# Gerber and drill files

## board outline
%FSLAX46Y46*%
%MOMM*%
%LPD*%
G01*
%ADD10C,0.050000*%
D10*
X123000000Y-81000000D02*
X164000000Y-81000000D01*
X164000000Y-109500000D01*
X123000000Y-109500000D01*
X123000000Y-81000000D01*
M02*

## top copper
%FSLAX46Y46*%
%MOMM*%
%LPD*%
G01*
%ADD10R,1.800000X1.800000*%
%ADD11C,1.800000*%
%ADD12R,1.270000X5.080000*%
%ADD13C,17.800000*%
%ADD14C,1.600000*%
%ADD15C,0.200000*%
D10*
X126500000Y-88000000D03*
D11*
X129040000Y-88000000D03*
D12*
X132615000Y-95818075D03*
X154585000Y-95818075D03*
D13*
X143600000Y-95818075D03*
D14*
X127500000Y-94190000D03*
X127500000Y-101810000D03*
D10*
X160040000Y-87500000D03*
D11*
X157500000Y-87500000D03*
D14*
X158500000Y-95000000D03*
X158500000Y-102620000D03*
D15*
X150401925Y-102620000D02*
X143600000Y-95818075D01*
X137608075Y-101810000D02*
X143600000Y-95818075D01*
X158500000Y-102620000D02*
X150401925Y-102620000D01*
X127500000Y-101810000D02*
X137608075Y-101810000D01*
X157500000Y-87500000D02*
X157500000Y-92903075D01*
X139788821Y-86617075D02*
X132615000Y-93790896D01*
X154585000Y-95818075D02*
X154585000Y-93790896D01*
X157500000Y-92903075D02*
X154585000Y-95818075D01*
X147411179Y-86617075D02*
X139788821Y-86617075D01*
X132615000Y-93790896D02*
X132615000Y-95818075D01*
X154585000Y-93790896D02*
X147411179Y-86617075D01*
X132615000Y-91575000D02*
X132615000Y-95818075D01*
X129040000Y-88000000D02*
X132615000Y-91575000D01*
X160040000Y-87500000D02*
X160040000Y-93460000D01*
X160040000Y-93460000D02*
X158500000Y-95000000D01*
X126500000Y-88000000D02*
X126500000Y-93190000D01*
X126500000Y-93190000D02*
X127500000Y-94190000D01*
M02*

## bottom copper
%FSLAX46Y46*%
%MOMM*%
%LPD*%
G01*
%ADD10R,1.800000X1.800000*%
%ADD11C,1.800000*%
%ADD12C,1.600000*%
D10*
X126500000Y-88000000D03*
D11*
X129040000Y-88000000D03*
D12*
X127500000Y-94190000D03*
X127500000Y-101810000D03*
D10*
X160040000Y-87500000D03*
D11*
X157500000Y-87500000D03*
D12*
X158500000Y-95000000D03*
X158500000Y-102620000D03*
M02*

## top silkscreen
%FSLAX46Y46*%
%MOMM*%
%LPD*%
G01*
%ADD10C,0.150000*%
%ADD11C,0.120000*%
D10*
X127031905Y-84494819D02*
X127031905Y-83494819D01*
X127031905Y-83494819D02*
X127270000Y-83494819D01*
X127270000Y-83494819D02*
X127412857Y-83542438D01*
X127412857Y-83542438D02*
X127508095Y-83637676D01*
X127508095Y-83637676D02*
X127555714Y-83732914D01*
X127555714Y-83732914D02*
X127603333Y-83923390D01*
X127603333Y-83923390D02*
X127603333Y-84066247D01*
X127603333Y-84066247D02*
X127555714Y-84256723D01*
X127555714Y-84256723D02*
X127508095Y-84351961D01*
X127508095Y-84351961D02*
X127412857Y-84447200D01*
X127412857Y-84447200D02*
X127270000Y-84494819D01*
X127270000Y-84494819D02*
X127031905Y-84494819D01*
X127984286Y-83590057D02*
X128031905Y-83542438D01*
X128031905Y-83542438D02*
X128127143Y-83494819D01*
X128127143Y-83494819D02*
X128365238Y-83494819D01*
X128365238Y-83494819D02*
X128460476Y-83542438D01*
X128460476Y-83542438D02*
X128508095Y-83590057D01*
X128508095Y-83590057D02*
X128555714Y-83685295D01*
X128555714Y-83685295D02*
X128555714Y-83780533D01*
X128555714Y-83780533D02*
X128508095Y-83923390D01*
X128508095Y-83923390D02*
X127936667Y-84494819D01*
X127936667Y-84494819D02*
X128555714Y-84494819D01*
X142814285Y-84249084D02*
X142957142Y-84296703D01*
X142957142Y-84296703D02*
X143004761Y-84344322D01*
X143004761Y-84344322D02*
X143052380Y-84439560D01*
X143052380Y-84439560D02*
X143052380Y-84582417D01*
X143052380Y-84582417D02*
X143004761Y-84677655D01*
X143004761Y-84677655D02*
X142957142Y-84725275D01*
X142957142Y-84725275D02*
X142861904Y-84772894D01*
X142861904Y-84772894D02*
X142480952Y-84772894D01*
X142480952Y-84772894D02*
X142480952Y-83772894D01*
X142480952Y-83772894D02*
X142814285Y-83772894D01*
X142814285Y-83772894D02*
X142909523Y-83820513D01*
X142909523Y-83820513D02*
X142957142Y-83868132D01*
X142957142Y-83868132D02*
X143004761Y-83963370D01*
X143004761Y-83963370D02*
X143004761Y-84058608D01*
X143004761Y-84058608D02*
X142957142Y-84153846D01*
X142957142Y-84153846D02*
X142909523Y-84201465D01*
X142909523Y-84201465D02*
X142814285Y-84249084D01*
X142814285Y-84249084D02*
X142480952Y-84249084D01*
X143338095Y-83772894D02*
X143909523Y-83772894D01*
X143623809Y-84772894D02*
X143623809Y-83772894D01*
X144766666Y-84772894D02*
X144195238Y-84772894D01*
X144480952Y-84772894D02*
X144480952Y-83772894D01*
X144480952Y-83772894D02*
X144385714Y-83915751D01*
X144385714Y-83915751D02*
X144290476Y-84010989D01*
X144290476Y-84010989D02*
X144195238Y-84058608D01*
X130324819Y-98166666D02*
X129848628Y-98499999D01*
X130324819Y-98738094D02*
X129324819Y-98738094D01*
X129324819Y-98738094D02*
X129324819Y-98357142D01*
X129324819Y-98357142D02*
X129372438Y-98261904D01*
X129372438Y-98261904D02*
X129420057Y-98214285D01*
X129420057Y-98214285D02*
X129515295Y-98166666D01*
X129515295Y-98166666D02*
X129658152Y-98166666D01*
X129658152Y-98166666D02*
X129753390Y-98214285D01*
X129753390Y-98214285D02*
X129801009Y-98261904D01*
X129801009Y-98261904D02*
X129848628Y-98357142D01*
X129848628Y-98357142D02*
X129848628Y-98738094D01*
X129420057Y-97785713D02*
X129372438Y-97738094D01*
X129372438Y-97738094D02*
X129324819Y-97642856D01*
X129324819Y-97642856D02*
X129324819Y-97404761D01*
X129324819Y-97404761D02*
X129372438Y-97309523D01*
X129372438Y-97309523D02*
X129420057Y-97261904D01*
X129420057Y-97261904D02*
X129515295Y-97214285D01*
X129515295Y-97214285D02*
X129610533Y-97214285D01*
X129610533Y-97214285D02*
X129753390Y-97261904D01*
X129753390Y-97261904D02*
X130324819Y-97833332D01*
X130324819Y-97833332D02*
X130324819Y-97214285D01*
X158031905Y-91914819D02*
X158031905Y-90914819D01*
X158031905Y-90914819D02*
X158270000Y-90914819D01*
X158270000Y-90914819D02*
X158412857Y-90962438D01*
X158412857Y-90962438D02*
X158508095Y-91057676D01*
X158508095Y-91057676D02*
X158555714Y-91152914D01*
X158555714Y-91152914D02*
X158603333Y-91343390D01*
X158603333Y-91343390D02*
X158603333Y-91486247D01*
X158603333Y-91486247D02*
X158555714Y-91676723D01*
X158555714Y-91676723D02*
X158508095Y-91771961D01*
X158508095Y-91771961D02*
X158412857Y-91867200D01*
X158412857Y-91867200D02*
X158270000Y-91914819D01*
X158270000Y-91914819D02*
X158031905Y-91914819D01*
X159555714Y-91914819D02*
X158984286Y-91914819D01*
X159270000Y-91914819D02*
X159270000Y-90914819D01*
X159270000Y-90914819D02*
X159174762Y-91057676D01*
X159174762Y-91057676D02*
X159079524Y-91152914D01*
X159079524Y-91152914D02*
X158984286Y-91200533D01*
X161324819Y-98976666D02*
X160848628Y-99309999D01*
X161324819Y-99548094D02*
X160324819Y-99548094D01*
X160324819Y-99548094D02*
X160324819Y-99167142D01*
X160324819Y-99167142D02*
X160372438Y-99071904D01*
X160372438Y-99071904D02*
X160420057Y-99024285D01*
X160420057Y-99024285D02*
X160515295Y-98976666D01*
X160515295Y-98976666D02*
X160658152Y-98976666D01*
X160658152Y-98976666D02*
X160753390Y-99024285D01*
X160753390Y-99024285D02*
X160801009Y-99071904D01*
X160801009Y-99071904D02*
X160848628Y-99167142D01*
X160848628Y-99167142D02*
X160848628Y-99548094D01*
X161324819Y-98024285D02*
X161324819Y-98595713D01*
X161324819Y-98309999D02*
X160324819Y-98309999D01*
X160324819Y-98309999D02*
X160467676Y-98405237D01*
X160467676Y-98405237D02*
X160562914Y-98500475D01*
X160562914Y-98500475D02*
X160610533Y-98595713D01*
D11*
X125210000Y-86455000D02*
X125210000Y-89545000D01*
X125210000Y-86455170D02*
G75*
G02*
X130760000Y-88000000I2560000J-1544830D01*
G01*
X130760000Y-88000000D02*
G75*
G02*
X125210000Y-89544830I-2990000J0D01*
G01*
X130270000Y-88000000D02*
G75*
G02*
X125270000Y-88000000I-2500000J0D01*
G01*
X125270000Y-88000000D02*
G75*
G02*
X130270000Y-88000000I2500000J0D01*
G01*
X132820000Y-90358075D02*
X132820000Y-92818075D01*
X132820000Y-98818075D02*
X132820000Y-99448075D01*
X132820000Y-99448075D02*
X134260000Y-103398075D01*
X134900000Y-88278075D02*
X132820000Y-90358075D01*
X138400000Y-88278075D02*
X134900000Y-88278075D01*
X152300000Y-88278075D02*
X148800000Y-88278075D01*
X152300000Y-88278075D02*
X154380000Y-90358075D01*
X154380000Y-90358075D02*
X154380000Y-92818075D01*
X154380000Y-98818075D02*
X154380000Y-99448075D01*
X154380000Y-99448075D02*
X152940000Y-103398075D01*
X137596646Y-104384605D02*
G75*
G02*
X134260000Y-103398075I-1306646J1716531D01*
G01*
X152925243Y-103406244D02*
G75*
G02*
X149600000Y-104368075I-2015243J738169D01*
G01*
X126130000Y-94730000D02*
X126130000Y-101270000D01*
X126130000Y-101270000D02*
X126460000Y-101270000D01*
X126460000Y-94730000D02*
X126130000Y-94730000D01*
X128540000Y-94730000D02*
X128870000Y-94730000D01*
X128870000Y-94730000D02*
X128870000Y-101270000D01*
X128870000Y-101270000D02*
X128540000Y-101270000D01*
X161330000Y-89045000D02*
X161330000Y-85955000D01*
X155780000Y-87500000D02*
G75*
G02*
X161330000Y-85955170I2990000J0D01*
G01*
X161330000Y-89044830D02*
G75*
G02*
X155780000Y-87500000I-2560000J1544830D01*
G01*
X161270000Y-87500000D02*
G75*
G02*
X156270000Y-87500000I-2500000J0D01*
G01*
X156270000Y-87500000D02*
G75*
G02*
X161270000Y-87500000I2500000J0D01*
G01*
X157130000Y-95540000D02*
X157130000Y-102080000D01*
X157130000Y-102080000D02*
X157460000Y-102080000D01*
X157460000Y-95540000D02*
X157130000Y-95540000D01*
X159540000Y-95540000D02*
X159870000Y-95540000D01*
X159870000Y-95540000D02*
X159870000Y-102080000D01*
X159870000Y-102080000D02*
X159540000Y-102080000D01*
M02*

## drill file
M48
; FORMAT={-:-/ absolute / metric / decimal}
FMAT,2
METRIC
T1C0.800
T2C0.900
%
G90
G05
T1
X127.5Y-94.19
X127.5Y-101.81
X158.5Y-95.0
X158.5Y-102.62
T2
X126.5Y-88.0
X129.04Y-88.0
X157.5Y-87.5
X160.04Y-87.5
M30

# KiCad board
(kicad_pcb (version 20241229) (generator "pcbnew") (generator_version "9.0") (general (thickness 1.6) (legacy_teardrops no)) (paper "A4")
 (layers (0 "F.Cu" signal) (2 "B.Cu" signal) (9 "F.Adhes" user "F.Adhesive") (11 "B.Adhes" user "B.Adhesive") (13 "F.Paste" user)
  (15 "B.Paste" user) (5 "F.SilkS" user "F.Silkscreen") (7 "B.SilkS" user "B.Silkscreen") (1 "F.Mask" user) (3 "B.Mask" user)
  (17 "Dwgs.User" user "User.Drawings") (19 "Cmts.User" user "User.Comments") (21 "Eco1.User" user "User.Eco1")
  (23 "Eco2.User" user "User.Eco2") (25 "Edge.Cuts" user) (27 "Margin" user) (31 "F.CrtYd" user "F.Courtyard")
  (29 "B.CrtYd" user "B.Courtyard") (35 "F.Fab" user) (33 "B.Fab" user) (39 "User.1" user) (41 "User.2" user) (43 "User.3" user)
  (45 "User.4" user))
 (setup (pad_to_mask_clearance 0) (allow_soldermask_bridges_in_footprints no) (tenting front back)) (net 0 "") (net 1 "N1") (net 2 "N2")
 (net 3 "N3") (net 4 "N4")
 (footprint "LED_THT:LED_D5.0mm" (layer "F.Cu") (at 126.5 88)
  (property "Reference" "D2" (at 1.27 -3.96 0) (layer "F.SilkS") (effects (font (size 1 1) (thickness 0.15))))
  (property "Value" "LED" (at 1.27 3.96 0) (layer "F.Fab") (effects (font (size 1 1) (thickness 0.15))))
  (fp_line (start -1.29 -1.545) (end -1.29 1.545) (stroke (width 0.12) (type solid)) (layer "F.SilkS"))
  (fp_arc (start -1.29 -1.54483) (mid 2.071779 -2.880495) (end 4.26 0) (stroke (width 0.12) (type solid)) (layer "F.SilkS"))
  (fp_arc (start 4.26 0) (mid 2.071779 2.880495) (end -1.29 1.54483) (stroke (width 0.12) (type solid)) (layer "F.SilkS"))
  (fp_circle (center 1.27 0) (end 3.77 0) (stroke (width 0.12) (type solid)) (fill no) (layer "F.SilkS"))
  (pad "1" thru_hole rect (at 0 0) (size 1.8 1.8) (drill 0.9) (layers "*.Cu" "*.Mask") (remove_unused_layers no) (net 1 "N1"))
  (pad "2" thru_hole circle (at 2.54 0) (size 1.8 1.8) (drill 0.9) (layers "*.Cu" "*.Mask") (remove_unused_layers no) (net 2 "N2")))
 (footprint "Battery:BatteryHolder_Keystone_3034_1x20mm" (layer "F.Cu") (at 143.6 95.818075)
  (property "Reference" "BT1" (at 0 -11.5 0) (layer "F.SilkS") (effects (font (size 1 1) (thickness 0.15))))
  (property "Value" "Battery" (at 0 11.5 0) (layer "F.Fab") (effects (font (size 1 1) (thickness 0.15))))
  (fp_line (start -10.78 -5.46) (end -10.78 -3) (stroke (width 0.12) (type solid)) (layer "F.SilkS"))
  (fp_line (start -10.78 3) (end -10.78 3.63) (stroke (width 0.12) (type solid)) (layer "F.SilkS"))
  (fp_line (start -10.78 3.63) (end -9.34 7.58) (stroke (width 0.12) (type solid)) (layer "F.SilkS"))
  (fp_line (start -8.7 -7.54) (end -10.78 -5.46) (stroke (width 0.12) (type solid)) (layer "F.SilkS"))
  (fp_line (start -5.2 -7.54) (end -8.7 -7.54) (stroke (width 0.12) (type solid)) (layer "F.SilkS"))
  (fp_line (start 8.7 -7.54) (end 5.2 -7.54) (stroke (width 0.12) (type solid)) (layer "F.SilkS"))
  (fp_line (start 8.7 -7.54) (end 10.78 -5.46) (stroke (width 0.12) (type solid)) (layer "F.SilkS"))
  (fp_line (start 10.78 -5.46) (end 10.78 -3) (stroke (width 0.12) (type solid)) (layer "F.SilkS"))
  (fp_line (start 10.78 3) (end 10.78 3.63) (stroke (width 0.12) (type solid)) (layer "F.SilkS"))
  (fp_line (start 10.78 3.63) (end 9.34 7.58) (stroke (width 0.12) (type solid)) (layer "F.SilkS"))
  (fp_arc (start -6.003354 8.56653) (mid -7.921654 8.918738) (end -9.34 7.58) (stroke (width 0.12) (type solid)) (layer "F.SilkS"))
  (fp_arc (start 9.325243 7.588169) (mid 7.90634 8.911668) (end 6 8.55) (stroke (width 0.12) (type solid)) (layer "F.SilkS"))
  (pad "1" smd rect (at -10.985 0) (size 1.27 5.08) (layers "F.Cu" "F.Mask" "F.Paste") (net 2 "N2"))
  (pad "1" smd rect (at 10.985 0) (size 1.27 5.08) (layers "F.Cu" "F.Mask" "F.Paste") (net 2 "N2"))
  (pad "2" smd circle (at 0 0) (size 17.8 17.8) (layers "F.Cu" "F.Mask") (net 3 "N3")))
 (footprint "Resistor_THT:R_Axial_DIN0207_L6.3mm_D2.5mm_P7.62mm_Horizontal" (layer "F.Cu") (at 127.5 94.19 -90)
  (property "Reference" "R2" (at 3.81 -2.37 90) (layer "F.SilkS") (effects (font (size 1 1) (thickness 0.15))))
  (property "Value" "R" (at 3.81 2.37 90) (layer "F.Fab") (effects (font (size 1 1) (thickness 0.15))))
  (fp_line (start 0.54 1.37) (end 7.08 1.37) (stroke (width 0.12) (type solid)) (layer "F.SilkS"))
  (fp_line (start 7.08 1.37) (end 7.08 1.04) (stroke (width 0.12) (type solid)) (layer "F.SilkS"))
  (fp_line (start 0.54 1.04) (end 0.54 1.37) (stroke (width 0.12) (type solid)) (layer "F.SilkS"))
  (fp_line (start 0.54 -1.04) (end 0.54 -1.37) (stroke (width 0.12) (type solid)) (layer "F.SilkS"))
  (fp_line (start 0.54 -1.37) (end 7.08 -1.37) (stroke (width 0.12) (type solid)) (layer "F.SilkS"))
  (fp_line (start 7.08 -1.37) (end 7.08 -1.04) (stroke (width 0.12) (type solid)) (layer "F.SilkS"))
  (pad "1" thru_hole circle (at 0 0 270) (size 1.6 1.6) (drill 0.8) (layers "*.Cu" "*.Mask") (remove_unused_layers no) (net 1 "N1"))
  (pad "2" thru_hole circle (at 7.62 0 270) (size 1.6 1.6) (drill 0.8) (layers "*.Cu" "*.Mask") (remove_unused_layers no) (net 3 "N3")))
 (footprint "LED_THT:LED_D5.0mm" (layer "F.Cu") (at 160.04 87.5 180)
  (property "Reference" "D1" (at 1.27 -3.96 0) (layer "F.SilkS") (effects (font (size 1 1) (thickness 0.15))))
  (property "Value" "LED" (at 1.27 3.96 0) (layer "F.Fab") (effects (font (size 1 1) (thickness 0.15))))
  (fp_line (start -1.29 -1.545) (end -1.29 1.545) (stroke (width 0.12) (type solid)) (layer "F.SilkS"))
  (fp_arc (start 4.26 0) (mid 2.071779 2.880495) (end -1.29 1.54483) (stroke (width 0.12) (type solid)) (layer "F.SilkS"))
  (fp_arc (start -1.29 -1.54483) (mid 2.071779 -2.880495) (end 4.26 0) (stroke (width 0.12) (type solid)) (layer "F.SilkS"))
  (fp_circle (center 1.27 0) (end 3.77 0) (stroke (width 0.12) (type solid)) (fill no) (layer "F.SilkS"))
  (pad "1" thru_hole rect (at 0 0 180) (size 1.8 1.8) (drill 0.9) (layers "*.Cu" "*.Mask") (remove_unused_layers no) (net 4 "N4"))
  (pad "2" thru_hole circle (at 2.54 0 180) (size 1.8 1.8) (drill 0.9) (layers "*.Cu" "*.Mask") (remove_unused_layers no) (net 2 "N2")))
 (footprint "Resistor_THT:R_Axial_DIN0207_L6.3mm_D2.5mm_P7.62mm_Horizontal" (layer "F.Cu") (at 158.5 95 -90)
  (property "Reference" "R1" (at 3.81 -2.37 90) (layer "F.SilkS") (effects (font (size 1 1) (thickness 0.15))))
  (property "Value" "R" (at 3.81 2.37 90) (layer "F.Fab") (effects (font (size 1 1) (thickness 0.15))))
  (fp_line (start 0.54 1.37) (end 7.08 1.37) (stroke (width 0.12) (type solid)) (layer "F.SilkS"))
  (fp_line (start 7.08 1.37) (end 7.08 1.04) (stroke (width 0.12) (type solid)) (layer "F.SilkS"))
  (fp_line (start 0.54 1.04) (end 0.54 1.37) (stroke (width 0.12) (type solid)) (layer "F.SilkS"))
  (fp_line (start 0.54 -1.04) (end 0.54 -1.37) (stroke (width 0.12) (type solid)) (layer "F.SilkS"))
  (fp_line (start 0.54 -1.37) (end 7.08 -1.37) (stroke (width 0.12) (type solid)) (layer "F.SilkS"))
  (fp_line (start 7.08 -1.37) (end 7.08 -1.04) (stroke (width 0.12) (type solid)) (layer "F.SilkS"))
  (pad "1" thru_hole circle (at 0 0 270) (size 1.6 1.6) (drill 0.8) (layers "*.Cu" "*.Mask") (remove_unused_layers no) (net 4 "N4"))
  (pad "2" thru_hole circle (at 7.62 0 270) (size 1.6 1.6) (drill 0.8) (layers "*.Cu" "*.Mask") (remove_unused_layers no) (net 3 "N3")))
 (gr_rect (start 123 81) (end 164 109.5) (stroke (width 0.05) (type default)) (fill no) (layer "Edge.Cuts"))
 (segment (start 150.401925 102.62) (end 143.6 95.818075) (width 0.2) (layer "F.Cu") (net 3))
 (segment (start 137.608075 101.81) (end 143.6 95.818075) (width 0.2) (layer "F.Cu") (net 3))
 (segment (start 158.5 102.62) (end 150.401925 102.62) (width 0.2) (layer "F.Cu") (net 3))
 (segment (start 127.5 101.81) (end 137.608075 101.81) (width 0.2) (layer "F.Cu") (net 3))
 (segment (start 157.5 87.5) (end 157.5 92.903075) (width 0.2) (layer "F.Cu") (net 2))
 (segment (start 139.788821 86.617075) (end 132.615 93.790896) (width 0.2) (layer "F.Cu") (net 2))
 (segment (start 154.585 95.818075) (end 154.585 93.790896) (width 0.2) (layer "F.Cu") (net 2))
 (segment (start 157.5 92.903075) (end 154.585 95.818075) (width 0.2) (layer "F.Cu") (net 2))
 (segment (start 147.411179 86.617075) (end 139.788821 86.617075) (width 0.2) (layer "F.Cu") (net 2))
 (segment (start 132.615 93.790896) (end 132.615 95.818075) (width 0.2) (layer "F.Cu") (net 2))
 (segment (start 154.585 93.790896) (end 147.411179 86.617075) (width 0.2) (layer "F.Cu") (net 2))
 (segment (start 132.615 91.575) (end 132.615 95.818075) (width 0.2) (layer "F.Cu") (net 2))
 (segment (start 129.04 88) (end 132.615 91.575) (width 0.2) (layer "F.Cu") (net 2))
 (segment (start 160.04 87.5) (end 160.04 93.46) (width 0.2) (layer "F.Cu") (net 4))
 (segment (start 160.04 93.46) (end 158.5 95) (width 0.2) (layer "F.Cu") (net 4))
 (segment (start 126.5 88) (end 126.5 93.19) (width 0.2) (layer "F.Cu") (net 1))
 (segment (start 126.5 93.19) (end 127.5 94.19) (width 0.2) (layer "F.Cu") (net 1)))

